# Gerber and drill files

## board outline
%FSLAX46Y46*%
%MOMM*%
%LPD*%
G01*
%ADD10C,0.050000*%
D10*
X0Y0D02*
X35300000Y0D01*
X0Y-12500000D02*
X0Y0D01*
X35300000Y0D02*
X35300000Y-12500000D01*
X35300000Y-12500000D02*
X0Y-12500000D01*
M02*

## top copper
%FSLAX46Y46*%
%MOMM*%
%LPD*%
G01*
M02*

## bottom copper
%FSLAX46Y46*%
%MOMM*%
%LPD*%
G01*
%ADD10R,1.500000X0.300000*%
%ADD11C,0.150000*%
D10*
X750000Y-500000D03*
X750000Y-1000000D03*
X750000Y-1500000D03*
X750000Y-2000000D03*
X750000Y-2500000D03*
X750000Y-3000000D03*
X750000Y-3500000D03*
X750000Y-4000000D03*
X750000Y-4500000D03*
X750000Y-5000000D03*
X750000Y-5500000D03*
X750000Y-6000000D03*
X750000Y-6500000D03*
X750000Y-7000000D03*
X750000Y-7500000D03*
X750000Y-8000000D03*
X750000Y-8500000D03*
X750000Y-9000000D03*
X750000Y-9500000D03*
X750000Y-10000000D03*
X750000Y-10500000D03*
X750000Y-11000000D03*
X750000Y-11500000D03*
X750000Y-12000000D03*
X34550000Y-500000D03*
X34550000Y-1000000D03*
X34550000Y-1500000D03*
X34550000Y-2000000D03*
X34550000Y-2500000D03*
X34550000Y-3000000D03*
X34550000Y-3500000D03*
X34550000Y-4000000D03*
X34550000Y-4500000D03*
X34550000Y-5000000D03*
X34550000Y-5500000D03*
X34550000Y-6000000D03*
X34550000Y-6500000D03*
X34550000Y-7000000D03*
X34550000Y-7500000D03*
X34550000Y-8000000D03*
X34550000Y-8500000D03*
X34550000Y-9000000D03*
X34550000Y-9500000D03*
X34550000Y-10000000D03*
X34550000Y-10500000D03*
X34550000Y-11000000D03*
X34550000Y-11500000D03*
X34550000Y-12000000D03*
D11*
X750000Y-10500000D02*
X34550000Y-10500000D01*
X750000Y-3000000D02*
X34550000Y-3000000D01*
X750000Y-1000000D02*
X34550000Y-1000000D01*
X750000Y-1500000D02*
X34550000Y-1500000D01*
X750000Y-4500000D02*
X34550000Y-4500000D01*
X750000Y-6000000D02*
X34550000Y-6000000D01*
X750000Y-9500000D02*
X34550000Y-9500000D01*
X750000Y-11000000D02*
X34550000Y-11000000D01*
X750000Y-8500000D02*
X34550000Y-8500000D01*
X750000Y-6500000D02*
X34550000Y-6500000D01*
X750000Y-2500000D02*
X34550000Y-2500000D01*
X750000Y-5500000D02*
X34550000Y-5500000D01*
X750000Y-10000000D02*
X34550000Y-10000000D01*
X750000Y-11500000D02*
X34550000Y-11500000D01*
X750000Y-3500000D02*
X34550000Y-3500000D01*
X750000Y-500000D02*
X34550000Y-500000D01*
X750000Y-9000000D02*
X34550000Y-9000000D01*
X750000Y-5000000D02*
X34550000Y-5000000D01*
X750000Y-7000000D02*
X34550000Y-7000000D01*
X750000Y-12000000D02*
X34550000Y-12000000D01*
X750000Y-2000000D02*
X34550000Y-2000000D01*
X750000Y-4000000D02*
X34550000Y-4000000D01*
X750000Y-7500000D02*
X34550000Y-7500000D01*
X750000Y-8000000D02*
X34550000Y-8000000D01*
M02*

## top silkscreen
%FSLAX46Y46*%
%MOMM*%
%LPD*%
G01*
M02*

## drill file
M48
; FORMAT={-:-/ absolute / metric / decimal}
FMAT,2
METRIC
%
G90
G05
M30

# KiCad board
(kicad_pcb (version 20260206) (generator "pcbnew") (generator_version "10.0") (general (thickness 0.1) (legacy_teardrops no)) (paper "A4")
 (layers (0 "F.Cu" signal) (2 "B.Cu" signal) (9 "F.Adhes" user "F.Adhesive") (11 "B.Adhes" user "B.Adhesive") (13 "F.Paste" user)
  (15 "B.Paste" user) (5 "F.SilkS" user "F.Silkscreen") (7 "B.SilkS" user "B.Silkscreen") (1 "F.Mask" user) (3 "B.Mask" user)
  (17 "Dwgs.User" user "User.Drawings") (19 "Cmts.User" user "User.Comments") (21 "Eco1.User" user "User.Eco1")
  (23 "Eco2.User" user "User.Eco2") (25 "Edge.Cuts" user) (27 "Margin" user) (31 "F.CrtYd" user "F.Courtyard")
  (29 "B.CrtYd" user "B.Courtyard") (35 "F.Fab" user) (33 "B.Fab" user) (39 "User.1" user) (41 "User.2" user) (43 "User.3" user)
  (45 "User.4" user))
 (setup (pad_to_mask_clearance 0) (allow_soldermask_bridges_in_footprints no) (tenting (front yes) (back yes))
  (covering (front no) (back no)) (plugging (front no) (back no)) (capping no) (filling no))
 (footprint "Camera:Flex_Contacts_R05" (layer "B.Cu") (at 0.75 6.25)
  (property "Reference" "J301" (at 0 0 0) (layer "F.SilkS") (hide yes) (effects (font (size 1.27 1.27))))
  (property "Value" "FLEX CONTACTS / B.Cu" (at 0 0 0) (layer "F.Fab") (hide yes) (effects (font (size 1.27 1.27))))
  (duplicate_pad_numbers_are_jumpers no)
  (pad "1" smd rect (at 0 -5.75) (size 1.5 0.3) (layers "B.Cu" "B.Mask") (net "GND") (thermal_bridge_angle 45))
  (pad "2" smd rect (at 0 -5.25) (size 1.5 0.3) (layers "B.Cu" "B.Mask") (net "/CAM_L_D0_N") (thermal_bridge_angle 45))
  (pad "3" smd rect (at 0 -4.75) (size 1.5 0.3) (layers "B.Cu" "B.Mask") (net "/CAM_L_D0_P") (thermal_bridge_angle 45))
  (pad "4" smd rect (at 0 -4.25) (size 1.5 0.3) (layers "B.Cu" "B.Mask") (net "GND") (thermal_bridge_angle 45))
  (pad "5" smd rect (at 0 -3.75) (size 1.5 0.3) (layers "B.Cu" "B.Mask") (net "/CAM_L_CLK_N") (thermal_bridge_angle 45))
  (pad "6" smd rect (at 0 -3.25) (size 1.5 0.3) (layers "B.Cu" "B.Mask") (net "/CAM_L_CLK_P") (thermal_bridge_angle 45))
  (pad "7" smd rect (at 0 -2.75) (size 1.5 0.3) (layers "B.Cu" "B.Mask") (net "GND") (thermal_bridge_angle 45))
  (pad "8" smd rect (at 0 -2.25) (size 1.5 0.3) (layers "B.Cu" "B.Mask") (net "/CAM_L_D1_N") (thermal_bridge_angle 45))
  (pad "9" smd rect (at 0 -1.75) (size 1.5 0.3) (layers "B.Cu" "B.Mask") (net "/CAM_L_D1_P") (thermal_bridge_angle 45))
  (pad "10" smd rect (at 0 -1.25) (size 1.5 0.3) (layers "B.Cu" "B.Mask") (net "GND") (thermal_bridge_angle 45))
  (pad "11" smd rect (at 0 -0.75) (size 1.5 0.3) (layers "B.Cu" "B.Mask") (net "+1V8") (thermal_bridge_angle 45))
  (pad "12" smd rect (at 0 -0.25) (size 1.5 0.3) (layers "B.Cu" "B.Mask") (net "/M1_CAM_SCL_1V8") (thermal_bridge_angle 45))
  (pad "13" smd rect (at 0 0.25) (size 1.5 0.3) (layers "B.Cu" "B.Mask") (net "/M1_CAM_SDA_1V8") (thermal_bridge_angle 45))
  (pad "14" smd rect (at 0 0.75) (size 1.5 0.3) (layers "B.Cu" "B.Mask") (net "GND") (thermal_bridge_angle 45))
  (pad "15" smd rect (at 0 1.25) (size 1.5 0.3) (layers "B.Cu" "B.Mask") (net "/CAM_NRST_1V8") (thermal_bridge_angle 45))
  (pad "16" smd rect (at 0 1.75) (size 1.5 0.3) (layers "B.Cu" "B.Mask") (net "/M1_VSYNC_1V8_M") (thermal_bridge_angle 45))
  (pad "17" smd rect (at 0 2.25) (size 1.5 0.3) (layers "B.Cu" "B.Mask") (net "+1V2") (thermal_bridge_angle 45))
  (pad "18" smd rect (at 0 2.75) (size 1.5 0.3) (layers "B.Cu" "B.Mask") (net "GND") (thermal_bridge_angle 45))
  (pad "19" smd rect (at 0 3.25) (size 1.5 0.3) (layers "B.Cu" "B.Mask") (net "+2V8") (thermal_bridge_angle 45))
  (pad "20" smd rect (at 0 3.75) (size 1.5 0.3) (layers "B.Cu" "B.Mask") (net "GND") (thermal_bridge_angle 45))
  (pad "21" smd rect (at 0 4.25) (size 1.5 0.3) (layers "B.Cu" "B.Mask") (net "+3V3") (thermal_bridge_angle 45))
  (pad "22" smd rect (at 0 4.75) (size 1.5 0.3) (layers "B.Cu" "B.Mask") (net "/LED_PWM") (thermal_bridge_angle 45))
  (pad "23" smd rect (at 0 5.25) (size 1.5 0.3) (layers "B.Cu" "B.Mask") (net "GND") (thermal_bridge_angle 45))
  (pad "24" smd rect (at 0 5.75) (size 1.5 0.3) (layers "B.Cu" "B.Mask") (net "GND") (thermal_bridge_angle 45)))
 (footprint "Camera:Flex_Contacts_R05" (layer "B.Cu") (at 34.55 6.25)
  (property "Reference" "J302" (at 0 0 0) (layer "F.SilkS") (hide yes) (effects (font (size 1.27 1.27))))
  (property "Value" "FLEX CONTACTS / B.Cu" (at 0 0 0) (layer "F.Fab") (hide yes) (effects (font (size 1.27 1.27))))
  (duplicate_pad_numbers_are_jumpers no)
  (pad "1" smd rect (at 0 -5.75) (size 1.5 0.3) (layers "B.Cu" "B.Mask") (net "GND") (thermal_bridge_angle 45))
  (pad "2" smd rect (at 0 -5.25) (size 1.5 0.3) (layers "B.Cu" "B.Mask") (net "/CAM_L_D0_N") (thermal_bridge_angle 45))
  (pad "3" smd rect (at 0 -4.75) (size 1.5 0.3) (layers "B.Cu" "B.Mask") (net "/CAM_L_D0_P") (thermal_bridge_angle 45))
  (pad "4" smd rect (at 0 -4.25) (size 1.5 0.3) (layers "B.Cu" "B.Mask") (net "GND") (thermal_bridge_angle 45))
  (pad "5" smd rect (at 0 -3.75) (size 1.5 0.3) (layers "B.Cu" "B.Mask") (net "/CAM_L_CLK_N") (thermal_bridge_angle 45))
  (pad "6" smd rect (at 0 -3.25) (size 1.5 0.3) (layers "B.Cu" "B.Mask") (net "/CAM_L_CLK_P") (thermal_bridge_angle 45))
  (pad "7" smd rect (at 0 -2.75) (size 1.5 0.3) (layers "B.Cu" "B.Mask") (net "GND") (thermal_bridge_angle 45))
  (pad "8" smd rect (at 0 -2.25) (size 1.5 0.3) (layers "B.Cu" "B.Mask") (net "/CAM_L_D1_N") (thermal_bridge_angle 45))
  (pad "9" smd rect (at 0 -1.75) (size 1.5 0.3) (layers "B.Cu" "B.Mask") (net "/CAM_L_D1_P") (thermal_bridge_angle 45))
  (pad "10" smd rect (at 0 -1.25) (size 1.5 0.3) (layers "B.Cu" "B.Mask") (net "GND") (thermal_bridge_angle 45))
  (pad "11" smd rect (at 0 -0.75) (size 1.5 0.3) (layers "B.Cu" "B.Mask") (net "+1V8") (thermal_bridge_angle 45))
  (pad "12" smd rect (at 0 -0.25) (size 1.5 0.3) (layers "B.Cu" "B.Mask") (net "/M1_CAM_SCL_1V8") (thermal_bridge_angle 45))
  (pad "13" smd rect (at 0 0.25) (size 1.5 0.3) (layers "B.Cu" "B.Mask") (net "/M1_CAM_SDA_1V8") (thermal_bridge_angle 45))
  (pad "14" smd rect (at 0 0.75) (size 1.5 0.3) (layers "B.Cu" "B.Mask") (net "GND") (thermal_bridge_angle 45))
  (pad "15" smd rect (at 0 1.25) (size 1.5 0.3) (layers "B.Cu" "B.Mask") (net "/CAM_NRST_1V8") (thermal_bridge_angle 45))
  (pad "16" smd rect (at 0 1.75) (size 1.5 0.3) (layers "B.Cu" "B.Mask") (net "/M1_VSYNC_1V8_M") (thermal_bridge_angle 45))
  (pad "17" smd rect (at 0 2.25) (size 1.5 0.3) (layers "B.Cu" "B.Mask") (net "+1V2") (thermal_bridge_angle 45))
  (pad "18" smd rect (at 0 2.75) (size 1.5 0.3) (layers "B.Cu" "B.Mask") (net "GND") (thermal_bridge_angle 45))
  (pad "19" smd rect (at 0 3.25) (size 1.5 0.3) (layers "B.Cu" "B.Mask") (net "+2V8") (thermal_bridge_angle 45))
  (pad "20" smd rect (at 0 3.75) (size 1.5 0.3) (layers "B.Cu" "B.Mask") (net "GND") (thermal_bridge_angle 45))
  (pad "21" smd rect (at 0 4.25) (size 1.5 0.3) (layers "B.Cu" "B.Mask") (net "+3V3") (thermal_bridge_angle 45))
  (pad "22" smd rect (at 0 4.75) (size 1.5 0.3) (layers "B.Cu" "B.Mask") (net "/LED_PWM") (thermal_bridge_angle 45))
  (pad "23" smd rect (at 0 5.25) (size 1.5 0.3) (layers "B.Cu" "B.Mask") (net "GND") (thermal_bridge_angle 45))
  (pad "24" smd rect (at 0 5.75) (size 1.5 0.3) (layers "B.Cu" "B.Mask") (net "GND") (thermal_bridge_angle 45)))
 (gr_line (start 0 0) (end 35.3 0) (stroke (width 0.05) (type default)) (layer "Edge.Cuts"))
 (gr_line (start 0 12.5) (end 0 0) (stroke (width 0.05) (type default)) (layer "Edge.Cuts"))
 (gr_line (start 35.3 0) (end 35.3 12.5) (stroke (width 0.05) (type default)) (layer "Edge.Cuts"))
 (gr_line (start 35.3 12.5) (end 0 12.5) (stroke (width 0.05) (type default)) (layer "Edge.Cuts"))
 (segment (start 0.75 10.5) (end 34.55 10.5) (width 0.15) (layer "B.Cu") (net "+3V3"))
 (segment (start 0.75 3) (end 34.55 3) (width 0.15) (layer "B.Cu") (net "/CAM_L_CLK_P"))
 (segment (start 0.75 1) (end 34.55 1) (width 0.15) (layer "B.Cu") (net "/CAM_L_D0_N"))
 (segment (start 0.75 1.5) (end 34.55 1.5) (width 0.15) (layer "B.Cu") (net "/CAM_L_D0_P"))
 (segment (start 0.75 4.5) (end 34.55 4.5) (width 0.15) (layer "B.Cu") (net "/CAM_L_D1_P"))
 (segment (start 0.75 6) (end 34.55 6) (width 0.15) (layer "B.Cu") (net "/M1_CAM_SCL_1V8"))
 (segment (start 0.75 9.5) (end 34.55 9.5) (width 0.15) (layer "B.Cu") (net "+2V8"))
 (segment (start 0.75 11) (end 34.55 11) (width 0.15) (layer "B.Cu") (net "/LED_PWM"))
 (segment (start 0.75 8.5) (end 34.55 8.5) (width 0.15) (layer "B.Cu") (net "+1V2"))
 (segment (start 0.75 6.5) (end 34.55 6.5) (width 0.15) (layer "B.Cu") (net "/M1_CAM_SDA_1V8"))
 (segment (start 0.75 2.5) (end 34.55 2.5) (width 0.15) (layer "B.Cu") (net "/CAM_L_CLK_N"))
 (segment (start 0.75 5.5) (end 34.55 5.5) (width 0.15) (layer "B.Cu") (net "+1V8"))
 (segment (start 0.75 10) (end 34.55 10) (width 0.15) (layer "B.Cu") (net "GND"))
 (segment (start 0.75 11.5) (end 34.55 11.5) (width 0.15) (layer "B.Cu") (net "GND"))
 (segment (start 0.75 3.5) (end 34.55 3.5) (width 0.15) (layer "B.Cu") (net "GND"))
 (segment (start 0.75 0.5) (end 34.55 0.5) (width 0.15) (layer "B.Cu") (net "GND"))
 (segment (start 0.75 9) (end 34.55 9) (width 0.15) (layer "B.Cu") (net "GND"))
 (segment (start 0.75 5) (end 34.55 5) (width 0.15) (layer "B.Cu") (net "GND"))
 (segment (start 0.75 7) (end 34.55 7) (width 0.15) (layer "B.Cu") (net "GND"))
 (segment (start 0.75 12) (end 34.55 12) (width 0.15) (layer "B.Cu") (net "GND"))
 (segment (start 0.75 2) (end 34.55 2) (width 0.15) (layer "B.Cu") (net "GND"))
 (segment (start 0.75 4) (end 34.55 4) (width 0.15) (layer "B.Cu") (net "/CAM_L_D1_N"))
 (segment (start 0.75 7.5) (end 34.55 7.5) (width 0.15) (layer "B.Cu") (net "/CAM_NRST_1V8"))
 (segment (start 0.75 8) (end 34.55 8) (width 0.15) (layer "B.Cu") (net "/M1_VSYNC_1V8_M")))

